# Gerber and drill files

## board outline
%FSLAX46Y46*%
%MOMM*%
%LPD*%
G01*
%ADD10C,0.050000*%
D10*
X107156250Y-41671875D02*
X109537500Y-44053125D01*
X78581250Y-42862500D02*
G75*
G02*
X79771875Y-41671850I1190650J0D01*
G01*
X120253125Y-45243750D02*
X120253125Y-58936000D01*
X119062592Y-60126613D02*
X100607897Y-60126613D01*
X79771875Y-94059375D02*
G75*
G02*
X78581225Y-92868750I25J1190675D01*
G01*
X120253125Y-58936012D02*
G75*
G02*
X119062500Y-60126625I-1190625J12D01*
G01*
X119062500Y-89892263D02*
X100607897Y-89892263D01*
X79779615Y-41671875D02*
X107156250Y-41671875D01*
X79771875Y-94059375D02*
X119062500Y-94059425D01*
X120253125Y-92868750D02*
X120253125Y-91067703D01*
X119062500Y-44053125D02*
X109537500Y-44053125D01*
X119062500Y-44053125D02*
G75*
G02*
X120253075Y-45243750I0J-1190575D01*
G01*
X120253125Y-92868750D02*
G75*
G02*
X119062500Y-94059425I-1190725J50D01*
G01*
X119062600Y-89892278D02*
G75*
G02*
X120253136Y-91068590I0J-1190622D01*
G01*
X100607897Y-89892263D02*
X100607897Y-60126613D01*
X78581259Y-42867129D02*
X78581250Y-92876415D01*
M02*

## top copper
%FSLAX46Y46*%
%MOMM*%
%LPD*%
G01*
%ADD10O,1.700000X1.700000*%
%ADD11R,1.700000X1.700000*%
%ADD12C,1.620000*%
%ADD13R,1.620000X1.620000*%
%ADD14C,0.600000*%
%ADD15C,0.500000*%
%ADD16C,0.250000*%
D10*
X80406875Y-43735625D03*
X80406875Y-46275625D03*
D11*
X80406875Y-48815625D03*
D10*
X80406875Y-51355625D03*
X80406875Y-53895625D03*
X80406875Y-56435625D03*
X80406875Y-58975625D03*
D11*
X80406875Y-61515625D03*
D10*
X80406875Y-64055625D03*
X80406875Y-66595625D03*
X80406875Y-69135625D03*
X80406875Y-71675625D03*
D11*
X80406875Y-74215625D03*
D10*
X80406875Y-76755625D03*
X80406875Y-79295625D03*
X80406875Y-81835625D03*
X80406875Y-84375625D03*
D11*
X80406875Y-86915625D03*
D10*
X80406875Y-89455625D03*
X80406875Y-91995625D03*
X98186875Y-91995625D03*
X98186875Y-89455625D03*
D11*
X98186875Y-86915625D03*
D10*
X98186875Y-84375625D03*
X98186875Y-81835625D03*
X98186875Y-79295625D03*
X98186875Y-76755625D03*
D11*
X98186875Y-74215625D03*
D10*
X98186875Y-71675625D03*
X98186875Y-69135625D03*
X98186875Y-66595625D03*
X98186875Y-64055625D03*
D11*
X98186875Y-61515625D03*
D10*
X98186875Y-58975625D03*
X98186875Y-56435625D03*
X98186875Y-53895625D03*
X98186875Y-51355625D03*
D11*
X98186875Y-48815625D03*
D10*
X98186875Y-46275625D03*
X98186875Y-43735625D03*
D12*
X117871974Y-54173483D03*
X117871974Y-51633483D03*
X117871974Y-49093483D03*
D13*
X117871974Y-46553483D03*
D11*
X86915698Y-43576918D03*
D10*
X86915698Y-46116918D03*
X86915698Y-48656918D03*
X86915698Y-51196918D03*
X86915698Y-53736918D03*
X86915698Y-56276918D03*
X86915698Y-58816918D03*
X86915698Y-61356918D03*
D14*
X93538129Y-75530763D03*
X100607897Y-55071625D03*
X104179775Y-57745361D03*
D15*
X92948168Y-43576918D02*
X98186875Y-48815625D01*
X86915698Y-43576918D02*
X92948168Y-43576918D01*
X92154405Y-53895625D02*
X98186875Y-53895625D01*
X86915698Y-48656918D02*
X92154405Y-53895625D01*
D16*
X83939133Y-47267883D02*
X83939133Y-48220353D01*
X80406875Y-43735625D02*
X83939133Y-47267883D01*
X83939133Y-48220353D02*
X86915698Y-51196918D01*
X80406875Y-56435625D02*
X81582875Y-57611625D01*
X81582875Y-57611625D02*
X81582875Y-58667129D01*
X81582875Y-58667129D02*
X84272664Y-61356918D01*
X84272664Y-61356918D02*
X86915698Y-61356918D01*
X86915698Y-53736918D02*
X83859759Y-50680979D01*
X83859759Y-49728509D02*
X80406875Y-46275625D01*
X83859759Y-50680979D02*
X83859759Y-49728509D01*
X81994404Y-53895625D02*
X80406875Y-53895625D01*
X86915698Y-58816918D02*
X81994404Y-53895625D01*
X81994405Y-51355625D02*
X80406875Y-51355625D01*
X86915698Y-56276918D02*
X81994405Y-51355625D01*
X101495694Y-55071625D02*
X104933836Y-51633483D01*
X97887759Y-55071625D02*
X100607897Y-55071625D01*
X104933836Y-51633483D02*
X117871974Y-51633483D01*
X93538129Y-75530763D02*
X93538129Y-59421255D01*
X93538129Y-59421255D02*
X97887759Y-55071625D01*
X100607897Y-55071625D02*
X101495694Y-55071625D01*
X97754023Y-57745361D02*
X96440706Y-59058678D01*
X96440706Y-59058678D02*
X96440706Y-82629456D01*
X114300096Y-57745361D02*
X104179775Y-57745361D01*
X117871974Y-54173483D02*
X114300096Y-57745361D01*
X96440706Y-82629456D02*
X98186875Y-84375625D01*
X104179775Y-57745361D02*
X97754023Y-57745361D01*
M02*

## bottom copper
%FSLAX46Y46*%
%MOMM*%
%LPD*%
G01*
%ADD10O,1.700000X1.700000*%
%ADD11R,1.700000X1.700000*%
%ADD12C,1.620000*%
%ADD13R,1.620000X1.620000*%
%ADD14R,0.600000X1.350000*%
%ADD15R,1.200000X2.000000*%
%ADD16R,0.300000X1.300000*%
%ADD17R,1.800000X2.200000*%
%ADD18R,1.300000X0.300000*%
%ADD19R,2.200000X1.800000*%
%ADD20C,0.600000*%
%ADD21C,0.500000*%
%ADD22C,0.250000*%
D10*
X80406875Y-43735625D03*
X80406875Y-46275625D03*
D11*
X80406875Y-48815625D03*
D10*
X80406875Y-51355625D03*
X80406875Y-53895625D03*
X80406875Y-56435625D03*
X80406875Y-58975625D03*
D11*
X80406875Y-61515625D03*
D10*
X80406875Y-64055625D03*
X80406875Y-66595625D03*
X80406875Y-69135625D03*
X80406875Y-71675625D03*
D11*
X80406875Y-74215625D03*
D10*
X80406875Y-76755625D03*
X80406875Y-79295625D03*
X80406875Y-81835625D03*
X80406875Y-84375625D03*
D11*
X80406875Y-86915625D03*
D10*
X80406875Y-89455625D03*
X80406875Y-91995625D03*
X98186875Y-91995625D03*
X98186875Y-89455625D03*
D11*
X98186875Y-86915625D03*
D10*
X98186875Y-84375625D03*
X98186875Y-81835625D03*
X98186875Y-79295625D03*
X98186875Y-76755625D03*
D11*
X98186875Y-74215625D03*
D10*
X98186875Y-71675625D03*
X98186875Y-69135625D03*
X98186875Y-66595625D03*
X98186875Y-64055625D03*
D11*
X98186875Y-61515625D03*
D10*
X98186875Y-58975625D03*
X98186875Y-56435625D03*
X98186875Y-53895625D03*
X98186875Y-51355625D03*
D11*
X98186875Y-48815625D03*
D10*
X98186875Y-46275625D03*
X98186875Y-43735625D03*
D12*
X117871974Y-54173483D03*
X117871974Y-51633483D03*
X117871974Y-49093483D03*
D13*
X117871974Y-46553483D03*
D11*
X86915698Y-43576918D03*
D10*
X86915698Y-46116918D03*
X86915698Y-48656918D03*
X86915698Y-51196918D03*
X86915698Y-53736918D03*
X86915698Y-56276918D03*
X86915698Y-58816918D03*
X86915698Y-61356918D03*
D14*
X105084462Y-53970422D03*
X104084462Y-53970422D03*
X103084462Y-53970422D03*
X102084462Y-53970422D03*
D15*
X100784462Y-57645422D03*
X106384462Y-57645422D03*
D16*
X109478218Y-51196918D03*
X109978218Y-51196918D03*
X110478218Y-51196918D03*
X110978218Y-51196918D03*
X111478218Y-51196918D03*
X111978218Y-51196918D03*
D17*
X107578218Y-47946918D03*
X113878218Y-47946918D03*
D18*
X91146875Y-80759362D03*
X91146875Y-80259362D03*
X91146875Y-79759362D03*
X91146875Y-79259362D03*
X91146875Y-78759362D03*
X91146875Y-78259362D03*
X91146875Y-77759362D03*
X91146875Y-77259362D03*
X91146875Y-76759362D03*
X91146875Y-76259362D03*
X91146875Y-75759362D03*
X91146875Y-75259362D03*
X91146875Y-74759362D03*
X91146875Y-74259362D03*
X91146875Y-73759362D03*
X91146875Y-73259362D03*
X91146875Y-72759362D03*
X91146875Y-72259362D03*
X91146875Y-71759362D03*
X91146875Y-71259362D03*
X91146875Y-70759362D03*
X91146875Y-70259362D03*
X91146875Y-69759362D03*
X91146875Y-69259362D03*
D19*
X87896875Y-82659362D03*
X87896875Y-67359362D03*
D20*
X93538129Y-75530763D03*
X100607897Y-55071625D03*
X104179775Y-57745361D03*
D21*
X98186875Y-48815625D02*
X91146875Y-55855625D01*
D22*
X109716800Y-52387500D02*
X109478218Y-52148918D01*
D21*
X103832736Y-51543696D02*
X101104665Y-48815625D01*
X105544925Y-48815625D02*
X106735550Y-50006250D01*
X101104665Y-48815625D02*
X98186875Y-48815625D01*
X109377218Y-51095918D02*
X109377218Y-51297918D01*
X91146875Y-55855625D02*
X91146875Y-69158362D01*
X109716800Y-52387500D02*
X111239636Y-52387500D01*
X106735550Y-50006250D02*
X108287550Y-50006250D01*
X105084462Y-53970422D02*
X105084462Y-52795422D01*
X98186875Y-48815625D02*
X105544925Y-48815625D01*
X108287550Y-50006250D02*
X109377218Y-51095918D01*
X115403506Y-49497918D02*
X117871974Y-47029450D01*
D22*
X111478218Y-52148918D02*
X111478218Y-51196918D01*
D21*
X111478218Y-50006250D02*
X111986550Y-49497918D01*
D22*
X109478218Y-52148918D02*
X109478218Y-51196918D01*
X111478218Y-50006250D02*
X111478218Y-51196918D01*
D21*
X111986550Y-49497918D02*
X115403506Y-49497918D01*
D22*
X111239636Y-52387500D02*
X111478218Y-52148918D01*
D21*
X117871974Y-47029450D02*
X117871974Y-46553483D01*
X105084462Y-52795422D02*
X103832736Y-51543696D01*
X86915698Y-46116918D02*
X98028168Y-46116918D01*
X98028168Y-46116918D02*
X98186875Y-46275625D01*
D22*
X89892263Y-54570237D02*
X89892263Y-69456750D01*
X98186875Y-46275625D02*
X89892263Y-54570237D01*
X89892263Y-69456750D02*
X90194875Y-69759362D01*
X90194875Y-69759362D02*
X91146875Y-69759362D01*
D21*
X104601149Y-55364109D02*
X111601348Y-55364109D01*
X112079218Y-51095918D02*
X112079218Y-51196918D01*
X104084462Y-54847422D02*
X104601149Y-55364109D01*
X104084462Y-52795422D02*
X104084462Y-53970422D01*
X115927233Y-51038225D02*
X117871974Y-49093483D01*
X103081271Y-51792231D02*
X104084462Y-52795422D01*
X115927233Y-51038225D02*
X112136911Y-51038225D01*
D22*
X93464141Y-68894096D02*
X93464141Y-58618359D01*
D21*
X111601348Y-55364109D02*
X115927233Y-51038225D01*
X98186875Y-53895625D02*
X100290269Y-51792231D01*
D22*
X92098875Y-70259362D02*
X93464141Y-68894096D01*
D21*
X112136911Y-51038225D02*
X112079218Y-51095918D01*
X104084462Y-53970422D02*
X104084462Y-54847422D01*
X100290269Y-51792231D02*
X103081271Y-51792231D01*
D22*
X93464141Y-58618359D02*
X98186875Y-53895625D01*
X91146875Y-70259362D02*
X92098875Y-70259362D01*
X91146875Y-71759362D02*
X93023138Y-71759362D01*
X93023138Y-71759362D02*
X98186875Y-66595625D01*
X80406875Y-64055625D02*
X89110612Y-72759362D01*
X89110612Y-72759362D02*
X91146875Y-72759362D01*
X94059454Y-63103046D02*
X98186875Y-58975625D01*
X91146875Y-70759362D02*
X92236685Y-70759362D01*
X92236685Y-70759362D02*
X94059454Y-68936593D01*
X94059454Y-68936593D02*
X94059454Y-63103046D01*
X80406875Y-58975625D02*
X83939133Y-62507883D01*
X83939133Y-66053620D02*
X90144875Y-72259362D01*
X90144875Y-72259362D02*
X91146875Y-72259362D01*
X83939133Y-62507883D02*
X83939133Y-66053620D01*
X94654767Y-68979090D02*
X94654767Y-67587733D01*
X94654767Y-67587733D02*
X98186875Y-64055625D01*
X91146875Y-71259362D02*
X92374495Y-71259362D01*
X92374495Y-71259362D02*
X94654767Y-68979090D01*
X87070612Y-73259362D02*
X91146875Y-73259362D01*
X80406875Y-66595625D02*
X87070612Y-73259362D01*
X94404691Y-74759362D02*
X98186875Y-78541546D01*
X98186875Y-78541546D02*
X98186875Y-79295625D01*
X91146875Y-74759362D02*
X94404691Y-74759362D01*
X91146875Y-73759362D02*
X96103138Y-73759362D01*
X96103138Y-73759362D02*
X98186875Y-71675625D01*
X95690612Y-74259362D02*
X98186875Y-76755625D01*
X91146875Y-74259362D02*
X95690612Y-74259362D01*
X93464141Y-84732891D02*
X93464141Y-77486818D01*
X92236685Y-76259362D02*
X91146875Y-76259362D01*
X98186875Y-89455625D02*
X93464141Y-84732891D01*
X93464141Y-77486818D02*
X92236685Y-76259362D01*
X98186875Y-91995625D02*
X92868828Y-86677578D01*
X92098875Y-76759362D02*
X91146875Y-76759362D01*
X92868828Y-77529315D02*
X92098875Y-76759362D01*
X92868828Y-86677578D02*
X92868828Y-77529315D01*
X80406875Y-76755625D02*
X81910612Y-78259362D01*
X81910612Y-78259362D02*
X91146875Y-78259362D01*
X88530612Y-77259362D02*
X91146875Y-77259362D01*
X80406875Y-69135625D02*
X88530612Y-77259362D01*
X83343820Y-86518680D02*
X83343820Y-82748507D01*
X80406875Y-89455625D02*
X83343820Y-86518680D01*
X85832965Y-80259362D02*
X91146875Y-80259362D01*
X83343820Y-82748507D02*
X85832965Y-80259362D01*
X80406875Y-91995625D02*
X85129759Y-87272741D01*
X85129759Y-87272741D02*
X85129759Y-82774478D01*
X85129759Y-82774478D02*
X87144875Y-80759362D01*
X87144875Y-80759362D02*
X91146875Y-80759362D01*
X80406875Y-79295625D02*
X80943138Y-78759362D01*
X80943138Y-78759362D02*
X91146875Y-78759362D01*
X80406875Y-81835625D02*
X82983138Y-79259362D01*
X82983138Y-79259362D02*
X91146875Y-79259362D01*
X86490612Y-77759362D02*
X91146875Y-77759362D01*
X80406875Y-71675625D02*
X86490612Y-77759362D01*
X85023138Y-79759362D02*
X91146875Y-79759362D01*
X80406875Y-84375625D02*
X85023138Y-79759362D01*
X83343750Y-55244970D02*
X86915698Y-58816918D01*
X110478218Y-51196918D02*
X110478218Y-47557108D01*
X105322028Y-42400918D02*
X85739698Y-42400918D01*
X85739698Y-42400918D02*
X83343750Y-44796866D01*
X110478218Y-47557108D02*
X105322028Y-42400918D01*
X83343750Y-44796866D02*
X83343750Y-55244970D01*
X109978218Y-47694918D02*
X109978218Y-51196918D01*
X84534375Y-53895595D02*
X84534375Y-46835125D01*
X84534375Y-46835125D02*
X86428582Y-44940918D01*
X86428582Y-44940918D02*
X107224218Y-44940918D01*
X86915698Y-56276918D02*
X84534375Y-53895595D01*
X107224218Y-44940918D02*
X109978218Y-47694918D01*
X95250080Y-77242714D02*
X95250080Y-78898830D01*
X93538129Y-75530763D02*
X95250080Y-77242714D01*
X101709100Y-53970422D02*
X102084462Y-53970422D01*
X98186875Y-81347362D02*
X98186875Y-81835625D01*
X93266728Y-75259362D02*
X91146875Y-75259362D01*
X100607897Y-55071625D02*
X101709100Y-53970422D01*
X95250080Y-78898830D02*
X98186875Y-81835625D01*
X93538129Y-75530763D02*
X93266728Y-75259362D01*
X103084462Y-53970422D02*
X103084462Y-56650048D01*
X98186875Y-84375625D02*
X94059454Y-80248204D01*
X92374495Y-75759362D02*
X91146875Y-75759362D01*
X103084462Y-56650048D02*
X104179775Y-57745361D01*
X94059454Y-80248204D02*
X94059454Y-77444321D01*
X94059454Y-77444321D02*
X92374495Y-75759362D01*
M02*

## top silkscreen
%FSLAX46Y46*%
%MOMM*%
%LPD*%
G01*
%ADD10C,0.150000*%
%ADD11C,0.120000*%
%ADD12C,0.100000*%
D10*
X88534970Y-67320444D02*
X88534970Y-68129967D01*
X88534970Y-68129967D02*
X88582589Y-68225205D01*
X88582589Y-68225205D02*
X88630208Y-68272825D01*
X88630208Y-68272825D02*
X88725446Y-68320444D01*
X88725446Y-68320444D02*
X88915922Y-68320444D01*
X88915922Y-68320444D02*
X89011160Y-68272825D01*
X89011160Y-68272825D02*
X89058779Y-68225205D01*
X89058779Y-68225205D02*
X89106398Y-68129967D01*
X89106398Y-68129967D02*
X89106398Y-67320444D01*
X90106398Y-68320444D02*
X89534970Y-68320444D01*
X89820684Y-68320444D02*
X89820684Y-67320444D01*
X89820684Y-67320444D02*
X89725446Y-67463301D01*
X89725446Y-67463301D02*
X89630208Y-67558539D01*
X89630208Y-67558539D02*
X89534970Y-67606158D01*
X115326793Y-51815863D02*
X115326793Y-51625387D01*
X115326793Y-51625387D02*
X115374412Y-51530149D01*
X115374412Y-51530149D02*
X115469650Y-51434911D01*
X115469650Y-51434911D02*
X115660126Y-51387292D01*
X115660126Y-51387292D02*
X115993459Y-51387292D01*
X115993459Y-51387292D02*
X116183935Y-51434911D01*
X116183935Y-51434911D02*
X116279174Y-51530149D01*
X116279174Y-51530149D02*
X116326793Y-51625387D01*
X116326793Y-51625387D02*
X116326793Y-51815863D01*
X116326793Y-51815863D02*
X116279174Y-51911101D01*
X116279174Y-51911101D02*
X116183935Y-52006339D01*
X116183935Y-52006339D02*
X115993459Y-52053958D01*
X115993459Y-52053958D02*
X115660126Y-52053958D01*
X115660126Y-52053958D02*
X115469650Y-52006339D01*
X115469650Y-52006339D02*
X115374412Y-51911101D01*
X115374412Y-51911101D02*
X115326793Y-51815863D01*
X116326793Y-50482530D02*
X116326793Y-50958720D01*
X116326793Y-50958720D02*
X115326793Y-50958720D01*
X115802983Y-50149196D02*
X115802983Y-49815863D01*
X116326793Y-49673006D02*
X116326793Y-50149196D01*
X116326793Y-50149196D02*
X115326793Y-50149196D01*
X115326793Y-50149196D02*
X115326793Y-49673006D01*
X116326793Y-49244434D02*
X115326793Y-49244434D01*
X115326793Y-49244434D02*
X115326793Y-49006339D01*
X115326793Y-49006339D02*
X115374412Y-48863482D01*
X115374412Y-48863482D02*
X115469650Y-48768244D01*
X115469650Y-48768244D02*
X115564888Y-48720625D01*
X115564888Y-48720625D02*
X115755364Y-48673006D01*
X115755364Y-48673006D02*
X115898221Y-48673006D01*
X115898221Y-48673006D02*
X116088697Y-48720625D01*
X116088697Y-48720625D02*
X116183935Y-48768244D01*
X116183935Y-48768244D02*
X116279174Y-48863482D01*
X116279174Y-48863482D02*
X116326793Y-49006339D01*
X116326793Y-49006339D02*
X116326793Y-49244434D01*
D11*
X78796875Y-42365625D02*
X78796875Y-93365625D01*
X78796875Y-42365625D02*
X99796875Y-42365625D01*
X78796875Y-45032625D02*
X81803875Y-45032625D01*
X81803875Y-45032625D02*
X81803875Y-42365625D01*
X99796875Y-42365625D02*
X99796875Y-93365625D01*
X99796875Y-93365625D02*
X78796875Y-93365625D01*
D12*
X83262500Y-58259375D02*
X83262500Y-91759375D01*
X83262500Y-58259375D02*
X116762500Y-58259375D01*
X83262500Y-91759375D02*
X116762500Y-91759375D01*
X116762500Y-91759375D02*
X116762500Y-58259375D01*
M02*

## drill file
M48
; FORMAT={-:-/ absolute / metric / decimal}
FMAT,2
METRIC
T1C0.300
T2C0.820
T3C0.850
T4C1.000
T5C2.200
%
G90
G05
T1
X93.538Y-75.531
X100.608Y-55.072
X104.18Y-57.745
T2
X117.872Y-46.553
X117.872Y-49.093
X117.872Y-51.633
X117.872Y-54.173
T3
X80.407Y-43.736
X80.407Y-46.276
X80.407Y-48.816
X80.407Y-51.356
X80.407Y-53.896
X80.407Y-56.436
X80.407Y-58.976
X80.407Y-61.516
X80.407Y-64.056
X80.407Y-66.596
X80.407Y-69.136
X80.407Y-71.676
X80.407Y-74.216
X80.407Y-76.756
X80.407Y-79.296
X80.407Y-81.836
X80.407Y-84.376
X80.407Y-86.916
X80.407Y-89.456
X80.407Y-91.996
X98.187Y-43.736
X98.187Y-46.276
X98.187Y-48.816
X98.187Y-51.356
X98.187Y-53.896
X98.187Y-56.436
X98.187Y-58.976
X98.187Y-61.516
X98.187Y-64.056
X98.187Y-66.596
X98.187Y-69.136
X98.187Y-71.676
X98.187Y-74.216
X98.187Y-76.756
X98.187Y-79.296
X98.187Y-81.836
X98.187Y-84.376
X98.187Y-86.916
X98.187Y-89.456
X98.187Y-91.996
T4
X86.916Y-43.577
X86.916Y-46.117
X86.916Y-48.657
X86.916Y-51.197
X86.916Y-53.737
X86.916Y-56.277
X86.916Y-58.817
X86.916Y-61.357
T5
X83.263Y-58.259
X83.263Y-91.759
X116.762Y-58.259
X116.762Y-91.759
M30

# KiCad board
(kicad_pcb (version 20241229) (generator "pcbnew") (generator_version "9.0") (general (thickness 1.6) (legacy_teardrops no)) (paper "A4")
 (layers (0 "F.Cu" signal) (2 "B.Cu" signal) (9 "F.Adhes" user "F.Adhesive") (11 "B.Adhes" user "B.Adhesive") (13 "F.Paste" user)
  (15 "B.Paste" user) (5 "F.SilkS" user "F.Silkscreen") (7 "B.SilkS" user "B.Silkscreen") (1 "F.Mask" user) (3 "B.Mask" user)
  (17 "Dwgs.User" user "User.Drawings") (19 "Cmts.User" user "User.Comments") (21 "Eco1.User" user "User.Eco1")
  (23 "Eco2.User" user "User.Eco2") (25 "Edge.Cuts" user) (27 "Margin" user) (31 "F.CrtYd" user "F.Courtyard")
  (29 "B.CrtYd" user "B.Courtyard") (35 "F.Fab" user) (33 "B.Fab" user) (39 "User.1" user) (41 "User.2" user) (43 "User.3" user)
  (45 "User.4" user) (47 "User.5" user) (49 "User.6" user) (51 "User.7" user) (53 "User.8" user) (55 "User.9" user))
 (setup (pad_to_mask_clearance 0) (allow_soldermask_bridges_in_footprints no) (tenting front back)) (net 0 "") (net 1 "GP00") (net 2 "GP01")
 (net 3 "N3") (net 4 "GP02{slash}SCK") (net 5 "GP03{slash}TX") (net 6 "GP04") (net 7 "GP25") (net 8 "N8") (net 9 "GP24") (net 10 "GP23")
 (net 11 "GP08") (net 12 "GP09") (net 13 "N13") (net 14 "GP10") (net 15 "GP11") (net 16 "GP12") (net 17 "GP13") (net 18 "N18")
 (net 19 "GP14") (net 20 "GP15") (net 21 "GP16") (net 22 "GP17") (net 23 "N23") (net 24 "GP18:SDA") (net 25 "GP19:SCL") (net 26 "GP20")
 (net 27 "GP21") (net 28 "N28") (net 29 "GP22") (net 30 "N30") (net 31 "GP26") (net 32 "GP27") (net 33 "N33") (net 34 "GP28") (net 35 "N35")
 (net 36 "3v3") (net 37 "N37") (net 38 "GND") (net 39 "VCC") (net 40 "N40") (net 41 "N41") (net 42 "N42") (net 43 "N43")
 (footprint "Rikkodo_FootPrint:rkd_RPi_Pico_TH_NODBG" (layer "F.Cu") (at 89.296875 67.865625)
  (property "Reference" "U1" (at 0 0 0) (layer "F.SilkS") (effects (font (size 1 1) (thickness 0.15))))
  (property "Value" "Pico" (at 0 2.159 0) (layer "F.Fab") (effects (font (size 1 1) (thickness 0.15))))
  (fp_line (start -10.5 -25.5) (end -10.5 25.5) (stroke (width 0.12) (type solid)) (layer "F.SilkS"))
  (fp_line (start -10.5 -25.5) (end 10.5 -25.5) (stroke (width 0.12) (type solid)) (layer "F.SilkS"))
  (fp_line (start -10.5 -22.833) (end -7.493 -22.833) (stroke (width 0.12) (type solid)) (layer "F.SilkS"))
  (fp_line (start -7.493 -22.833) (end -7.493 -25.5) (stroke (width 0.12) (type solid)) (layer "F.SilkS"))
  (fp_line (start 10.5 -25.5) (end 10.5 25.5) (stroke (width 0.12) (type solid)) (layer "F.SilkS"))
  (fp_line (start 10.5 25.5) (end -10.5 25.5) (stroke (width 0.12) (type solid)) (layer "F.SilkS"))
  (pad "1" thru_hole oval (at -8.89 -24.13) (size 1.7 1.7) (drill 0.85) (layers "*.Cu" "*.Mask") (remove_unused_layers no) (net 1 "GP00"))
  (pad "2" thru_hole oval (at -8.89 -21.59) (size 1.7 1.7) (drill 0.85) (layers "*.Cu" "*.Mask") (remove_unused_layers no) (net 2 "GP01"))
  (pad "3" thru_hole rect (at -8.89 -19.05) (size 1.7 1.7) (drill 0.85) (layers "*.Cu" "*.Mask") (remove_unused_layers no) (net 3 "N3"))
  (pad "4" thru_hole oval (at -8.89 -16.51) (size 1.7 1.7) (drill 0.85) (layers "*.Cu" "*.Mask") (remove_unused_layers no)
   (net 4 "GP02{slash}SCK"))
  (pad "5" thru_hole oval (at -8.89 -13.97) (size 1.7 1.7) (drill 0.85) (layers "*.Cu" "*.Mask") (remove_unused_layers no)
   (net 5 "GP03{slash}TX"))
  (pad "6" thru_hole oval (at -8.89 -11.43) (size 1.7 1.7) (drill 0.85) (layers "*.Cu" "*.Mask") (remove_unused_layers no) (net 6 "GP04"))
  (pad "7" thru_hole oval (at -8.89 -8.89) (size 1.7 1.7) (drill 0.85) (layers "*.Cu" "*.Mask") (remove_unused_layers no) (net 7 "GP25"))
  (pad "8" thru_hole rect (at -8.89 -6.35) (size 1.7 1.7) (drill 0.85) (layers "*.Cu" "*.Mask") (remove_unused_layers no) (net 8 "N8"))
  (pad "9" thru_hole oval (at -8.89 -3.81) (size 1.7 1.7) (drill 0.85) (layers "*.Cu" "*.Mask") (remove_unused_layers no) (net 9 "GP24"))
  (pad "10" thru_hole oval (at -8.89 -1.27) (size 1.7 1.7) (drill 0.85) (layers "*.Cu" "*.Mask") (remove_unused_layers no) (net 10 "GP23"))
  (pad "11" thru_hole oval (at -8.89 1.27) (size 1.7 1.7) (drill 0.85) (layers "*.Cu" "*.Mask") (remove_unused_layers no) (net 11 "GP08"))
  (pad "12" thru_hole oval (at -8.89 3.81) (size 1.7 1.7) (drill 0.85) (layers "*.Cu" "*.Mask") (remove_unused_layers no) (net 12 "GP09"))
  (pad "13" thru_hole rect (at -8.89 6.35) (size 1.7 1.7) (drill 0.85) (layers "*.Cu" "*.Mask") (remove_unused_layers no) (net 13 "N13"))
  (pad "14" thru_hole oval (at -8.89 8.89) (size 1.7 1.7) (drill 0.85) (layers "*.Cu" "*.Mask") (remove_unused_layers no) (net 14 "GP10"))
  (pad "15" thru_hole oval (at -8.89 11.43) (size 1.7 1.7) (drill 0.85) (layers "*.Cu" "*.Mask") (remove_unused_layers no) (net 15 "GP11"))
  (pad "16" thru_hole oval (at -8.89 13.97) (size 1.7 1.7) (drill 0.85) (layers "*.Cu" "*.Mask") (remove_unused_layers no) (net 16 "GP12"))
  (pad "17" thru_hole oval (at -8.89 16.51) (size 1.7 1.7) (drill 0.85) (layers "*.Cu" "*.Mask") (remove_unused_layers no) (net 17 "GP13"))
  (pad "18" thru_hole rect (at -8.89 19.05) (size 1.7 1.7) (drill 0.85) (layers "*.Cu" "*.Mask") (remove_unused_layers no) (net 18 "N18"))
  (pad "19" thru_hole oval (at -8.89 21.59) (size 1.7 1.7) (drill 0.85) (layers "*.Cu" "*.Mask") (remove_unused_layers no) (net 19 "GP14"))
  (pad "20" thru_hole oval (at -8.89 24.13) (size 1.7 1.7) (drill 0.85) (layers "*.Cu" "*.Mask") (remove_unused_layers no) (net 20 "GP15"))
  (pad "21" thru_hole oval (at 8.89 24.13) (size 1.7 1.7) (drill 0.85) (layers "*.Cu" "*.Mask") (remove_unused_layers no) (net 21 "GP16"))
  (pad "22" thru_hole oval (at 8.89 21.59) (size 1.7 1.7) (drill 0.85) (layers "*.Cu" "*.Mask") (remove_unused_layers no) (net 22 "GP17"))
  (pad "23" thru_hole rect (at 8.89 19.05) (size 1.7 1.7) (drill 0.85) (layers "*.Cu" "*.Mask") (remove_unused_layers no) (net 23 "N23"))
  (pad "24" thru_hole oval (at 8.89 16.51) (size 1.7 1.7) (drill 0.85) (layers "*.Cu" "*.Mask") (remove_unused_layers no)
   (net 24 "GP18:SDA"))
  (pad "25" thru_hole oval (at 8.89 13.97) (size 1.7 1.7) (drill 0.85) (layers "*.Cu" "*.Mask") (remove_unused_layers no)
   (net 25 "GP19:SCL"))
  (pad "26" thru_hole oval (at 8.89 11.43) (size 1.7 1.7) (drill 0.85) (layers "*.Cu" "*.Mask") (remove_unused_layers no) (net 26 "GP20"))
  (pad "27" thru_hole oval (at 8.89 8.89) (size 1.7 1.7) (drill 0.85) (layers "*.Cu" "*.Mask") (remove_unused_layers no) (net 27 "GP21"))
  (pad "28" thru_hole rect (at 8.89 6.35) (size 1.7 1.7) (drill 0.85) (layers "*.Cu" "*.Mask") (remove_unused_layers no) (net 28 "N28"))
  (pad "29" thru_hole oval (at 8.89 3.81) (size 1.7 1.7) (drill 0.85) (layers "*.Cu" "*.Mask") (remove_unused_layers no) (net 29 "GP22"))
  (pad "30" thru_hole oval (at 8.89 1.27) (size 1.7 1.7) (drill 0.85) (layers "*.Cu" "*.Mask") (remove_unused_layers no) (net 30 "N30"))
  (pad "31" thru_hole oval (at 8.89 -1.27) (size 1.7 1.7) (drill 0.85) (layers "*.Cu" "*.Mask") (remove_unused_layers no) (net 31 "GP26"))
  (pad "32" thru_hole oval (at 8.89 -3.81) (size 1.7 1.7) (drill 0.85) (layers "*.Cu" "*.Mask") (remove_unused_layers no) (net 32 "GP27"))
  (pad "33" thru_hole rect (at 8.89 -6.35) (size 1.7 1.7) (drill 0.85) (layers "*.Cu" "*.Mask") (remove_unused_layers no) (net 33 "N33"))
  (pad "34" thru_hole oval (at 8.89 -8.89) (size 1.7 1.7) (drill 0.85) (layers "*.Cu" "*.Mask") (remove_unused_layers no) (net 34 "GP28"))
  (pad "35" thru_hole oval (at 8.89 -11.43) (size 1.7 1.7) (drill 0.85) (layers "*.Cu" "*.Mask") (remove_unused_layers no) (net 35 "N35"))
  (pad "36" thru_hole oval (at 8.89 -13.97) (size 1.7 1.7) (drill 0.85) (layers "*.Cu" "*.Mask") (remove_unused_layers no) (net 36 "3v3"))
  (pad "37" thru_hole oval (at 8.89 -16.51) (size 1.7 1.7) (drill 0.85) (layers "*.Cu" "*.Mask") (remove_unused_layers no) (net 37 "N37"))
  (pad "38" thru_hole rect (at 8.89 -19.05) (size 1.7 1.7) (drill 0.85) (layers "*.Cu" "*.Mask") (remove_unused_layers no) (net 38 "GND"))
  (pad "39" thru_hole oval (at 8.89 -21.59) (size 1.7 1.7) (drill 0.85) (layers "*.Cu" "*.Mask") (remove_unused_layers no) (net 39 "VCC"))
  (pad "40" thru_hole oval (at 8.89 -24.13) (size 1.7 1.7) (drill 0.85) (layers "*.Cu" "*.Mask") (remove_unused_layers no) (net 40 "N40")))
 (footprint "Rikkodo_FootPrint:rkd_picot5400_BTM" (layer "F.Cu") (at 100.0125 75.009375)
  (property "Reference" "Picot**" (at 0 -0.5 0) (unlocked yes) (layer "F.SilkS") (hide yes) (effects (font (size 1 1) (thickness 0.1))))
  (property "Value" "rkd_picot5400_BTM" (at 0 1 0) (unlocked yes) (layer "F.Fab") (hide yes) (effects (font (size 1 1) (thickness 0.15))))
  (fp_line (start -16.75 -16.75) (end -16.75 16.75) (stroke (width 0.1) (type default)) (layer "F.SilkS"))
  (fp_line (start -16.75 -16.75) (end 16.75 -16.75) (stroke (width 0.1) (type default)) (layer "F.SilkS"))
  (fp_line (start -16.75 16.75) (end 16.75 16.75) (stroke (width 0.1) (type default)) (layer "F.SilkS"))
  (fp_line (start 16.75 16.75) (end 16.75 -16.75) (stroke (width 0.1) (type default)) (layer "F.SilkS"))
  (pad "" np_thru_hole circle (at -16.75 -16.75) (size 2.2 2.2) (drill 2.2) (layers "*.Cu" "*.Mask"))
  (pad "" np_thru_hole circle (at -16.75 16.75) (size 2.2 2.2) (drill 2.2) (layers "*.Cu" "*.Mask"))
  (pad "" np_thru_hole circle (at 16.75 -16.75) (size 2.2 2.2) (drill 2.2) (layers "*.Cu" "*.Mask"))
  (pad "" np_thru_hole circle (at 16.75 16.75) (size 2.2 2.2) (drill 2.2) (layers "*.Cu" "*.Mask")))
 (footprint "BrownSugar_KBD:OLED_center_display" (layer "F.Cu") (at 99.371974 50.363483 90)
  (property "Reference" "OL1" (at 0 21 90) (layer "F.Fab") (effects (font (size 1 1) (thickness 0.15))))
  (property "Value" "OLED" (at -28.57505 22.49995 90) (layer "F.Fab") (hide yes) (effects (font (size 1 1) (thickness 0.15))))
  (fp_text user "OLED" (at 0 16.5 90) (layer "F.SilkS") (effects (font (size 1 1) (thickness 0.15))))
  (pad "1" thru_hole circle (at -3.81 18.5 90) (size 1.62 1.62) (drill 0.82) (layers "*.Cu" "*.Mask") (remove_unused_layers no)
   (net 24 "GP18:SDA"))
  (pad "2" thru_hole circle (at -1.27 18.5 90) (size 1.62 1.62) (drill 0.82) (layers "*.Cu" "*.Mask") (remove_unused_layers no)
   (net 25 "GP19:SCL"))
  (pad "3" thru_hole circle (at 1.27 18.5 90) (size 1.62 1.62) (drill 0.82) (layers "*.Cu" "*.Mask") (remove_unused_layers no)
   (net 36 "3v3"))
  (pad "4" thru_hole rect (at 3.81 18.5 90) (size 1.62 1.62) (drill 0.82) (layers "*.Cu" "*.Mask") (remove_unused_layers no) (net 38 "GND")))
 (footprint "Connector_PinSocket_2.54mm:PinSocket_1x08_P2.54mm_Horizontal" (layer "B.Cu") (at 86.915698 43.576918 180)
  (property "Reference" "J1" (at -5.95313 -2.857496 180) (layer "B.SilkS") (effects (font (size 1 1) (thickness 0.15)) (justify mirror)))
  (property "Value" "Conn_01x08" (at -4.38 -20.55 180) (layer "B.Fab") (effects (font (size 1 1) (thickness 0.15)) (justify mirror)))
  (pad "1" thru_hole rect (at 0 0 180) (size 1.7 1.7) (drill 1) (layers "*.Cu" "*.Mask") (remove_unused_layers no) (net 38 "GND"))
  (pad "2" thru_hole oval (at 0 -2.54 180) (size 1.7 1.7) (drill 1) (layers "*.Cu" "*.Mask") (remove_unused_layers no) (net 39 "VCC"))
  (pad "3" thru_hole oval (at 0 -5.08 180) (size 1.7 1.7) (drill 1) (layers "*.Cu" "*.Mask") (remove_unused_layers no) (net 36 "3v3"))
  (pad "4" thru_hole oval (at 0 -7.62 180) (size 1.7 1.7) (drill 1) (layers "*.Cu" "*.Mask") (remove_unused_layers no) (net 1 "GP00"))
  (pad "5" thru_hole oval (at 0 -10.16 180) (size 1.7 1.7) (drill 1) (layers "*.Cu" "*.Mask") (remove_unused_layers no) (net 2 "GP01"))
  (pad "6" thru_hole oval (at 0 -12.7 180) (size 1.7 1.7) (drill 1) (layers "*.Cu" "*.Mask") (remove_unused_layers no)
   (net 4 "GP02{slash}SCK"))
  (pad "7" thru_hole oval (at 0 -15.24 180) (size 1.7 1.7) (drill 1) (layers "*.Cu" "*.Mask") (remove_unused_layers no)
   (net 5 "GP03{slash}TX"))
  (pad "8" thru_hole oval (at 0 -17.78 180) (size 1.7 1.7) (drill 1) (layers "*.Cu" "*.Mask") (remove_unused_layers no) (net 6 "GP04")))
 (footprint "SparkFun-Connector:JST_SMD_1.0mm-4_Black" (layer "B.Cu") (at 103.584462 53.970422 180)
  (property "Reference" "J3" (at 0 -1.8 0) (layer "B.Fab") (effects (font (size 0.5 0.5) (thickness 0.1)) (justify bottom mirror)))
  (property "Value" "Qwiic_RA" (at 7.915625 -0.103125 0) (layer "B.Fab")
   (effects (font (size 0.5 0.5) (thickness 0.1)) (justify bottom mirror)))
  (pad "1" smd rect (at -1.5 0 180) (size 0.6 1.35) (layers "B.Cu" "B.Mask" "B.Paste") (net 38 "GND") (thermal_bridge_angle 0))
  (pad "2" smd rect (at -0.5 0 180) (size 0.6 1.35) (layers "B.Cu" "B.Mask" "B.Paste") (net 36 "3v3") (thermal_bridge_angle 0))
  (pad "3" smd rect (at 0.5 0 180) (size 0.6 1.35) (layers "B.Cu" "B.Mask" "B.Paste") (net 24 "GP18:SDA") (thermal_bridge_angle 0))
  (pad "4" smd rect (at 1.5 0 180) (size 0.6 1.35) (layers "B.Cu" "B.Mask" "B.Paste") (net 25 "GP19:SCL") (thermal_bridge_angle 0))
  (pad "NC1" smd rect (at 2.8 -3.675 180) (size 1.2 2) (layers "B.Cu" "B.Mask" "B.Paste") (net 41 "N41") (thermal_bridge_angle 0))
  (pad "NC2" smd rect (at -2.8 -3.675 180) (size 1.2 2) (layers "B.Cu" "B.Mask" "B.Paste") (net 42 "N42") (thermal_bridge_angle 0)))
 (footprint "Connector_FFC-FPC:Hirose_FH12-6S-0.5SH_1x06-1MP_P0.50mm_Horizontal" (layer "B.Cu") (at 110.728218 49.346918)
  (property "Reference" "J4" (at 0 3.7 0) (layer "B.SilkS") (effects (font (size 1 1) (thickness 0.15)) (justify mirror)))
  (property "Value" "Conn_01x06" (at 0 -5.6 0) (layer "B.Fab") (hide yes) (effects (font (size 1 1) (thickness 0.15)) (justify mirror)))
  (pad "1" smd rect (at -1.25 1.85) (size 0.3 1.3) (layers "B.Cu" "B.Mask" "B.Paste") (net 38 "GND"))
  (pad "2" smd rect (at -0.75 1.85) (size 0.3 1.3) (layers "B.Cu" "B.Mask" "B.Paste") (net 4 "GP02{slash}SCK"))
  (pad "3" smd rect (at -0.25 1.85) (size 0.3 1.3) (layers "B.Cu" "B.Mask" "B.Paste") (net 5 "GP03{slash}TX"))
  (pad "4" smd rect (at 0.25 1.85) (size 0.3 1.3) (layers "B.Cu" "B.Mask" "B.Paste") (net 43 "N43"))
  (pad "5" smd rect (at 0.75 1.85) (size 0.3 1.3) (layers "B.Cu" "B.Mask" "B.Paste") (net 38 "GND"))
  (pad "6" smd rect (at 1.25 1.85) (size 0.3 1.3) (layers "B.Cu" "B.Mask" "B.Paste") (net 36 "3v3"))
  (pad "MP" smd rect (at -3.15 -1.4) (size 1.8 2.2) (layers "B.Cu" "B.Mask" "B.Paste"))
  (pad "MP" smd rect (at 3.15 -1.4) (size 1.8 2.2) (layers "B.Cu" "B.Mask" "B.Paste")))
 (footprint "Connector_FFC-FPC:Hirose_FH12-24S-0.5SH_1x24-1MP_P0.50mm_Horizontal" (layer "B.Cu") (at 89.296875 75.009362 90)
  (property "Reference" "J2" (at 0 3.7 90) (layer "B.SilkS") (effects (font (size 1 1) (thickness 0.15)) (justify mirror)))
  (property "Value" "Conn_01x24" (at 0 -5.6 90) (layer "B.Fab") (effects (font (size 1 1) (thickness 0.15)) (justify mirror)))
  (pad "1" smd rect (at -5.75 1.85 90) (size 0.3 1.3) (layers "B.Cu" "B.Mask" "B.Paste") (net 20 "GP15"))
  (pad "2" smd rect (at -5.25 1.85 90) (size 0.3 1.3) (layers "B.Cu" "B.Mask" "B.Paste") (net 19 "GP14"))
  (pad "3" smd rect (at -4.75 1.85 90) (size 0.3 1.3) (layers "B.Cu" "B.Mask" "B.Paste") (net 17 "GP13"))
  (pad "4" smd rect (at -4.25 1.85 90) (size 0.3 1.3) (layers "B.Cu" "B.Mask" "B.Paste") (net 16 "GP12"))
  (pad "5" smd rect (at -3.75 1.85 90) (size 0.3 1.3) (layers "B.Cu" "B.Mask" "B.Paste") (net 15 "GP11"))
  (pad "6" smd rect (at -3.25 1.85 90) (size 0.3 1.3) (layers "B.Cu" "B.Mask" "B.Paste") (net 14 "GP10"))
  (pad "7" smd rect (at -2.75 1.85 90) (size 0.3 1.3) (layers "B.Cu" "B.Mask" "B.Paste") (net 12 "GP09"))
  (pad "8" smd rect (at -2.25 1.85 90) (size 0.3 1.3) (layers "B.Cu" "B.Mask" "B.Paste") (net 11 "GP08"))
  (pad "9" smd rect (at -1.75 1.85 90) (size 0.3 1.3) (layers "B.Cu" "B.Mask" "B.Paste") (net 21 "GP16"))
  (pad "10" smd rect (at -1.25 1.85 90) (size 0.3 1.3) (layers "B.Cu" "B.Mask" "B.Paste") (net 22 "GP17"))
  (pad "11" smd rect (at -0.75 1.85 90) (size 0.3 1.3) (layers "B.Cu" "B.Mask" "B.Paste") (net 24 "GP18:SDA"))
  (pad "12" smd rect (at -0.25 1.85 90) (size 0.3 1.3) (layers "B.Cu" "B.Mask" "B.Paste") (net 25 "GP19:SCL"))
  (pad "13" smd rect (at 0.25 1.85 90) (size 0.3 1.3) (layers "B.Cu" "B.Mask" "B.Paste") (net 26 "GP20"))
  (pad "14" smd rect (at 0.75 1.85 90) (size 0.3 1.3) (layers "B.Cu" "B.Mask" "B.Paste") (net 27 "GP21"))
  (pad "15" smd rect (at 1.25 1.85 90) (size 0.3 1.3) (layers "B.Cu" "B.Mask" "B.Paste") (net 29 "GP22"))
  (pad "16" smd rect (at 1.75 1.85 90) (size 0.3 1.3) (layers "B.Cu" "B.Mask" "B.Paste") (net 10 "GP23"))
  (pad "17" smd rect (at 2.25 1.85 90) (size 0.3 1.3) (layers "B.Cu" "B.Mask" "B.Paste") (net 9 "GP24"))
  (pad "18" smd rect (at 2.75 1.85 90) (size 0.3 1.3) (layers "B.Cu" "B.Mask" "B.Paste") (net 7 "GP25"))
  (pad "19" smd rect (at 3.25 1.85 90) (size 0.3 1.3) (layers "B.Cu" "B.Mask" "B.Paste") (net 31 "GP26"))
  (pad "20" smd rect (at 3.75 1.85 90) (size 0.3 1.3) (layers "B.Cu" "B.Mask" "B.Paste") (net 32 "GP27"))
  (pad "21" smd rect (at 4.25 1.85 90) (size 0.3 1.3) (layers "B.Cu" "B.Mask" "B.Paste") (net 34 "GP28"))
  (pad "22" smd rect (at 4.75 1.85 90) (size 0.3 1.3) (layers "B.Cu" "B.Mask" "B.Paste") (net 36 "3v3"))
  (pad "23" smd rect (at 5.25 1.85 90) (size 0.3 1.3) (layers "B.Cu" "B.Mask" "B.Paste") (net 39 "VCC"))
  (pad "24" smd rect (at 5.75 1.85 90) (size 0.3 1.3) (layers "B.Cu" "B.Mask" "B.Paste") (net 38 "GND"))
  (pad "MP" smd rect (at -7.65 -1.4 90) (size 1.8 2.2) (layers "B.Cu" "B.Mask" "B.Paste"))
  (pad "MP" smd rect (at 7.65 -1.4 90) (size 1.8 2.2) (layers "B.Cu" "B.Mask" "B.Paste")))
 (gr_line (start 107.15625 41.671875) (end 109.5375 44.053125) (stroke (width 0.05) (type default)) (layer "Edge.Cuts"))
 (gr_arc (start 78.58125 42.8625) (mid 78.929974 42.020592) (end 79.771875 41.671875) (stroke (width 0.05) (type default))
  (layer "Edge.Cuts"))
 (gr_line (start 120.253125 45.24375) (end 120.253125 58.936) (stroke (width 0.05) (type default)) (layer "Edge.Cuts"))
 (gr_line (start 119.062592 60.126613) (end 100.607897 60.126613) (stroke (width 0.05) (type default)) (layer "Edge.Cuts"))
 (gr_arc (start 79.771875 94.059375) (mid 78.929974 93.710643) (end 78.58125 92.86875) (stroke (width 0.05) (type default))
  (layer "Edge.Cuts"))
 (gr_arc (start 120.253125 58.936012) (mid 119.904395 59.777903) (end 119.0625 60.126637) (stroke (width 0.05) (type default))
  (layer "Edge.Cuts"))
 (gr_line (start 119.0625 89.892263) (end 100.607897 89.892263) (stroke (width 0.05) (type default)) (layer "Edge.Cuts"))
 (gr_line (start 79.779615 41.671875) (end 107.15625 41.671875) (stroke (width 0.05) (type default)) (layer "Edge.Cuts"))
 (gr_line (start 79.771875 94.059375) (end 119.0625 94.059425) (stroke (width 0.05) (type default)) (layer "Edge.Cuts"))
 (gr_line (start 120.253125 92.86875) (end 120.253125 91.067703) (stroke (width 0.05) (type default)) (layer "Edge.Cuts"))
 (gr_line (start 119.0625 44.053125) (end 109.5375 44.053125) (stroke (width 0.05) (type default)) (layer "Edge.Cuts"))
 (gr_arc (start 119.0625 44.053125) (mid 119.904417 44.401848) (end 120.253125 45.24375) (stroke (width 0.05) (type default))
  (layer "Edge.Cuts"))
 (gr_arc (start 120.253125 92.86875) (mid 119.904381 93.710617) (end 119.0625 94.059375) (stroke (width 0.05) (type default))
  (layer "Edge.Cuts"))
 (gr_arc (start 119.0626 89.892278) (mid 119.899422 90.235959) (end 120.253125 91.06859) (stroke (width 0.05) (type default))
  (layer "Edge.Cuts"))
 (gr_line (start 100.607897 89.892263) (end 100.607897 60.126613) (stroke (width 0.05) (type default)) (layer "Edge.Cuts"))
 (gr_line (start 78.581259 42.867129) (end 78.58125 92.876415) (stroke (width 0.05) (type default)) (layer "Edge.Cuts"))
 (segment (start 92.948168 43.576918) (end 98.186875 48.815625) (width 0.5) (layer "F.Cu") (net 38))
 (segment (start 86.915698 43.576918) (end 92.948168 43.576918) (width 0.5) (layer "F.Cu") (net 38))
 (segment (start 98.186875 48.815625) (end 91.146875 55.855625) (width 0.5) (layer "B.Cu") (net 38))
 (segment (start 109.7168 52.3875) (end 109.478218 52.148918) (width 0.25) (layer "B.Cu") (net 38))
 (segment (start 103.832736 51.543696) (end 101.104665 48.815625) (width 0.5) (layer "B.Cu") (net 38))
 (segment (start 105.544925 48.815625) (end 106.73555 50.00625) (width 0.5) (layer "B.Cu") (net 38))
 (segment (start 101.104665 48.815625) (end 98.186875 48.815625) (width 0.5) (layer "B.Cu") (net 38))
 (segment (start 109.377218 51.095918) (end 109.377218 51.297918) (width 0.5) (layer "B.Cu") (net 38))
 (segment (start 91.146875 55.855625) (end 91.146875 69.158362) (width 0.5) (layer "B.Cu") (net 38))
 (segment (start 109.7168 52.3875) (end 111.239636 52.3875) (width 0.5) (layer "B.Cu") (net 38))
 (segment (start 106.73555 50.00625) (end 108.28755 50.00625) (width 0.5) (layer "B.Cu") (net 38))
 (segment (start 105.084462 53.970422) (end 105.084462 52.795422) (width 0.5) (layer "B.Cu") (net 38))
 (segment (start 98.186875 48.815625) (end 105.544925 48.815625) (width 0.5) (layer "B.Cu") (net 38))
 (segment (start 108.28755 50.00625) (end 109.377218 51.095918) (width 0.5) (layer "B.Cu") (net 38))
 (segment (start 115.403506 49.497918) (end 117.871974 47.02945) (width 0.5) (layer "B.Cu") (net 38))
 (segment (start 111.478218 52.148918) (end 111.478218 51.196918) (width 0.25) (layer "B.Cu") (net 38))
 (segment (start 111.478218 50.00625) (end 111.98655 49.497918) (width 0.5) (layer "B.Cu") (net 38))
 (segment (start 109.478218 52.148918) (end 109.478218 51.196918) (width 0.25) (layer "B.Cu") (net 38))
 (segment (start 111.478218 50.00625) (end 111.478218 51.196918) (width 0.25) (layer "B.Cu") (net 38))
 (segment (start 111.98655 49.497918) (end 115.403506 49.497918) (width 0.5) (layer "B.Cu") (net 38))
 (segment (start 111.239636 52.3875) (end 111.478218 52.148918) (width 0.25) (layer "B.Cu") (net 38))
 (segment (start 117.871974 47.02945) (end 117.871974 46.553483) (width 0.5) (layer "B.Cu") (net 38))
 (segment (start 105.084462 52.795422) (end 103.832736 51.543696) (width 0.5) (layer "B.Cu") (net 38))
 (segment (start 86.915698 46.116918) (end 98.028168 46.116918) (width 0.5) (layer "B.Cu") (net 39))
 (segment (start 98.028168 46.116918) (end 98.186875 46.275625) (width 0.5) (layer "B.Cu") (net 39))
 (segment (start 89.892263 54.570237) (end 89.892263 69.45675) (width 0.25) (layer "B.Cu") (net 39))
 (segment (start 98.186875 46.275625) (end 89.892263 54.570237) (width 0.25) (layer "B.Cu") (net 39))
 (segment (start 89.892263 69.45675) (end 90.194875 69.759362) (width 0.25) (layer "B.Cu") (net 39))
 (segment (start 90.194875 69.759362) (end 91.146875 69.759362) (width 0.25) (layer "B.Cu") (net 39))
 (segment (start 92.154405 53.895625) (end 98.186875 53.895625) (width 0.5) (layer "F.Cu") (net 36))
 (segment (start 86.915698 48.656918) (end 92.154405 53.895625) (width 0.5) (layer "F.Cu") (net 36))
 (segment (start 104.601149 55.364109) (end 111.601348 55.364109) (width 0.5) (layer "B.Cu") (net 36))
 (segment (start 112.079218 51.095918) (end 112.079218 51.196918) (width 0.5) (layer "B.Cu") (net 36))
 (segment (start 104.084462 54.847422) (end 104.601149 55.364109) (width 0.5) (layer "B.Cu") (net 36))
 (segment (start 104.084462 52.795422) (end 104.084462 53.970422) (width 0.5) (layer "B.Cu") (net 36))
 (segment (start 115.927233 51.038225) (end 117.871974 49.093483) (width 0.5) (layer "B.Cu") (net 36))
 (segment (start 103.081271 51.792231) (end 104.084462 52.795422) (width 0.5) (layer "B.Cu") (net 36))
 (segment (start 115.927233 51.038225) (end 112.136911 51.038225) (width 0.5) (layer "B.Cu") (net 36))
 (segment (start 93.464141 68.894096) (end 93.464141 58.618359) (width 0.25) (layer "B.Cu") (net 36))
 (segment (start 111.601348 55.364109) (end 115.927233 51.038225) (width 0.5) (layer "B.Cu") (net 36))
 (segment (start 98.186875 53.895625) (end 100.290269 51.792231) (width 0.5) (layer "B.Cu") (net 36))
 (segment (start 92.098875 70.259362) (end 93.464141 68.894096) (width 0.25) (layer "B.Cu") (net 36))
 (segment (start 112.136911 51.038225) (end 112.079218 51.095918) (width 0.5) (layer "B.Cu") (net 36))
 (segment (start 104.084462 53.970422) (end 104.084462 54.847422) (width 0.5) (layer "B.Cu") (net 36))
 (segment (start 100.290269 51.792231) (end 103.081271 51.792231) (width 0.5) (layer "B.Cu") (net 36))
 (segment (start 93.464141 58.618359) (end 98.186875 53.895625) (width 0.25) (layer "B.Cu") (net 36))
 (segment (start 91.146875 70.259362) (end 92.098875 70.259362) (width 0.25) (layer "B.Cu") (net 36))
 (segment (start 91.146875 71.759362) (end 93.023138 71.759362) (width 0.25) (layer "B.Cu") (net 31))
 (segment (start 93.023138 71.759362) (end 98.186875 66.595625) (width 0.25) (layer "B.Cu") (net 31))
 (segment (start 80.406875 64.055625) (end 89.110612 72.759362) (width 0.25) (layer "B.Cu") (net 9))
 (segment (start 89.110612 72.759362) (end 91.146875 72.759362) (width 0.25) (layer "B.Cu") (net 9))
 (segment (start 94.059454 63.103046) (end 98.186875 58.975625) (width 0.25) (layer "B.Cu") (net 34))
 (segment (start 91.146875 70.759362) (end 92.236685 70.759362) (width 0.25) (layer "B.Cu") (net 34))
 (segment (start 92.236685 70.759362) (end 94.059454 68.936593) (width 0.25) (layer "B.Cu") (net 34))
 (segment (start 94.059454 68.936593) (end 94.059454 63.103046) (width 0.25) (layer "B.Cu") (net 34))
 (segment (start 80.406875 58.975625) (end 83.939133 62.507883) (width 0.25) (layer "B.Cu") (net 7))
 (segment (start 83.939133 66.05362) (end 90.144875 72.259362) (width 0.25) (layer "B.Cu") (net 7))
 (segment (start 90.144875 72.259362) (end 91.146875 72.259362) (width 0.25) (layer "B.Cu") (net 7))
 (segment (start 83.939133 62.507883) (end 83.939133 66.05362) (width 0.25) (layer "B.Cu") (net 7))
 (segment (start 94.654767 68.97909) (end 94.654767 67.587733) (width 0.25) (layer "B.Cu") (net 32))
 (segment (start 94.654767 67.587733) (end 98.186875 64.055625) (width 0.25) (layer "B.Cu") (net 32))
 (segment (start 91.146875 71.259362) (end 92.374495 71.259362) (width 0.25) (layer "B.Cu") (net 32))
 (segment (start 92.374495 71.259362) (end 94.654767 68.97909) (width 0.25) (layer "B.Cu") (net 32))
 (segment (start 87.070612 73.259362) (end 91.146875 73.259362) (width 0.25) (layer "B.Cu") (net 10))
 (segment (start 80.406875 66.595625) (end 87.070612 73.259362) (width 0.25) (layer "B.Cu") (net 10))
 (segment (start 94.404691 74.759362) (end 98.186875 78.541546) (width 0.25) (layer "B.Cu") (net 26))
 (segment (start 98.186875 78.541546) (end 98.186875 79.295625) (width 0.25) (layer "B.Cu") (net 26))
 (segment (start 91.146875 74.759362) (end 94.404691 74.759362) (width 0.25) (layer "B.Cu") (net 26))
 (segment (start 91.146875 73.759362) (end 96.103138 73.759362) (width 0.25) (layer "B.Cu") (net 29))
 (segment (start 96.103138 73.759362) (end 98.186875 71.675625) (width 0.25) (layer "B.Cu") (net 29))
 (segment (start 95.690612 74.259362) (end 98.186875 76.755625) (width 0.25) (layer "B.Cu") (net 27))
 (segment (start 91.146875 74.259362) (end 95.690612 74.259362) (width 0.25) (layer "B.Cu") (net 27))
 (segment (start 93.464141 84.732891) (end 93.464141 77.486818) (width 0.25) (layer "B.Cu") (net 22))
 (segment (start 92.236685 76.259362) (end 91.146875 76.259362) (width 0.25) (layer "B.Cu") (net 22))
 (segment (start 98.186875 89.455625) (end 93.464141 84.732891) (width 0.25) (layer "B.Cu") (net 22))
 (segment (start 93.464141 77.486818) (end 92.236685 76.259362) (width 0.25) (layer "B.Cu") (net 22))
 (segment (start 98.186875 91.995625) (end 92.868828 86.677578) (width 0.25) (layer "B.Cu") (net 21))
 (segment (start 92.098875 76.759362) (end 91.146875 76.759362) (width 0.25) (layer "B.Cu") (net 21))
 (segment (start 92.868828 77.529315) (end 92.098875 76.759362) (width 0.25) (layer "B.Cu") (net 21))
 (segment (start 92.868828 86.677578) (end 92.868828 77.529315) (width 0.25) (layer "B.Cu") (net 21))
 (segment (start 80.406875 76.755625) (end 81.910612 78.259362) (width 0.25) (layer "B.Cu") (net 14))
 (segment (start 81.910612 78.259362) (end 91.146875 78.259362) (width 0.25) (layer "B.Cu") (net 14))
 (segment (start 88.530612 77.259362) (end 91.146875 77.259362) (width 0.25) (layer "B.Cu") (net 11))
 (segment (start 80.406875 69.135625) (end 88.530612 77.259362) (width 0.25) (layer "B.Cu") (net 11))
 (segment (start 83.34382 86.51868) (end 83.34382 82.748507) (width 0.25) (layer "B.Cu") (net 19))
 (segment (start 80.406875 89.455625) (end 83.34382 86.51868) (width 0.25) (layer "B.Cu") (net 19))
 (segment (start 85.832965 80.259362) (end 91.146875 80.259362) (width 0.25) (layer "B.Cu") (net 19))
 (segment (start 83.34382 82.748507) (end 85.832965 80.259362) (width 0.25) (layer "B.Cu") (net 19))
 (segment (start 80.406875 91.995625) (end 85.129759 87.272741) (width 0.25) (layer "B.Cu") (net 20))
 (segment (start 85.129759 87.272741) (end 85.129759 82.774478) (width 0.25) (layer "B.Cu") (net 20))
 (segment (start 85.129759 82.774478) (end 87.144875 80.759362) (width 0.25) (layer "B.Cu") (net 20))
 (segment (start 87.144875 80.759362) (end 91.146875 80.759362) (width 0.25) (layer "B.Cu") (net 20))
 (segment (start 80.406875 79.295625) (end 80.943138 78.759362) (width 0.25) (layer "B.Cu") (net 15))
 (segment (start 80.943138 78.759362) (end 91.146875 78.759362) (width 0.25) (layer "B.Cu") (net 15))
 (segment (start 80.406875 81.835625) (end 82.983138 79.259362) (width 0.25) (layer "B.Cu") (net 16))
 (segment (start 82.983138 79.259362) (end 91.146875 79.259362) (width 0.25) (layer "B.Cu") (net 16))
 (segment (start 86.490612 77.759362) (end 91.146875 77.759362) (width 0.25) (layer "B.Cu") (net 12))
 (segment (start 80.406875 71.675625) (end 86.490612 77.759362) (width 0.25) (layer "B.Cu") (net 12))
 (segment (start 85.023138 79.759362) (end 91.146875 79.759362) (width 0.25) (layer "B.Cu") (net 17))
 (segment (start 80.406875 84.375625) (end 85.023138 79.759362) (width 0.25) (layer "B.Cu") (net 17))
 (segment (start 83.939133 47.267883) (end 83.939133 48.220353) (width 0.25) (layer "F.Cu") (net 1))
 (segment (start 80.406875 43.735625) (end 83.939133 47.267883) (width 0.25) (layer "F.Cu") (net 1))
 (segment (start 83.939133 48.220353) (end 86.915698 51.196918) (width 0.25) (layer "F.Cu") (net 1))
 (segment (start 80.406875 56.435625) (end 81.582875 57.611625) (width 0.25) (layer "F.Cu") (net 6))
 (segment (start 81.582875 57.611625) (end 81.582875 58.667129) (width 0.25) (layer "F.Cu") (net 6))
 (segment (start 81.582875 58.667129) (end 84.272664 61.356918) (width 0.25) (layer "F.Cu") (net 6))
 (segment (start 84.272664 61.356918) (end 86.915698 61.356918) (width 0.25) (layer "F.Cu") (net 6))
 (segment (start 86.915698 53.736918) (end 83.859759 50.680979) (width 0.25) (layer "F.Cu") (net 2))
 (segment (start 83.859759 49.728509) (end 80.406875 46.275625) (width 0.25) (layer "F.Cu") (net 2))
 (segment (start 83.859759 50.680979) (end 83.859759 49.728509) (width 0.25) (layer "F.Cu") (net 2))
 (segment (start 81.994404 53.895625) (end 80.406875 53.895625) (width 0.25) (layer "F.Cu") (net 5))
 (segment (start 86.915698 58.816918) (end 81.994404 53.895625) (width 0.25) (layer "F.Cu") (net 5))
 (segment (start 83.34375 55.24497) (end 86.915698 58.816918) (width 0.25) (layer "B.Cu") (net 5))
 (segment (start 110.478218 51.196918) (end 110.478218 47.557108) (width 0.25) (layer "B.Cu") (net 5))
 (segment (start 105.322028 42.400918) (end 85.739698 42.400918) (width 0.25) (layer "B.Cu") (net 5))
 (segment (start 85.739698 42.400918) (end 83.34375 44.796866) (width 0.25) (layer "B.Cu") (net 5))
 (segment (start 110.478218 47.557108) (end 105.322028 42.400918) (width 0.25) (layer "B.Cu") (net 5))
 (segment (start 83.34375 44.796866) (end 83.34375 55.24497) (width 0.25) (layer "B.Cu") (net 5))
 (segment (start 81.994405 51.355625) (end 80.406875 51.355625) (width 0.25) (layer "F.Cu") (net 4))
 (segment (start 86.915698 56.276918) (end 81.994405 51.355625) (width 0.25) (layer "F.Cu") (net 4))
 (segment (start 109.978218 47.694918) (end 109.978218 51.196918) (width 0.25) (layer "B.Cu") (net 4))
 (segment (start 84.534375 53.895595) (end 84.534375 46.835125) (width 0.25) (layer "B.Cu") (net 4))
 (segment (start 84.534375 46.835125) (end 86.428582 44.940918) (width 0.25) (layer "B.Cu") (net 4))
 (segment (start 86.428582 44.940918) (end 107.224218 44.940918) (width 0.25) (layer "B.Cu") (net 4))
 (segment (start 86.915698 56.276918) (end 84.534375 53.895595) (width 0.25) (layer "B.Cu") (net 4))
 (segment (start 107.224218 44.940918) (end 109.978218 47.694918) (width 0.25) (layer "B.Cu") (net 4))
 (segment (start 101.495694 55.071625) (end 104.933836 51.633483) (width 0.25) (layer "F.Cu") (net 25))
 (segment (start 97.887759 55.071625) (end 100.607897 55.071625) (width 0.25) (layer "F.Cu") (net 25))
 (segment (start 104.933836 51.633483) (end 117.871974 51.633483) (width 0.25) (layer "F.Cu") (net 25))
 (segment (start 93.538129 75.530763) (end 93.538129 59.421255) (width 0.25) (layer "F.Cu") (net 25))
 (segment (start 93.538129 59.421255) (end 97.887759 55.071625) (width 0.25) (layer "F.Cu") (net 25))
 (segment (start 100.607897 55.071625) (end 101.495694 55.071625) (width 0.25) (layer "F.Cu") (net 25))
 (via (at 93.538129 75.530763) (size 0.6) (drill 0.3) (layers "F.Cu" "B.Cu") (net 25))
 (via (at 100.607897 55.071625) (size 0.6) (drill 0.3) (layers "F.Cu" "B.Cu") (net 25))
 (segment (start 95.25008 77.242714) (end 95.25008 78.89883) (width 0.25) (layer "B.Cu") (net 25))
 (segment (start 93.538129 75.530763) (end 95.25008 77.242714) (width 0.25) (layer "B.Cu") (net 25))
 (segment (start 101.7091 53.970422) (end 102.084462 53.970422) (width 0.25) (layer "B.Cu") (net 25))
 (segment (start 98.186875 81.347362) (end 98.186875 81.835625) (width 0.25) (layer "B.Cu") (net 25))
 (segment (start 93.266728 75.259362) (end 91.146875 75.259362) (width 0.25) (layer "B.Cu") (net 25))
 (segment (start 100.607897 55.071625) (end 101.7091 53.970422) (width 0.25) (layer "B.Cu") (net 25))
 (segment (start 95.25008 78.89883) (end 98.186875 81.835625) (width 0.25) (layer "B.Cu") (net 25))
 (segment (start 93.538129 75.530763) (end 93.266728 75.259362) (width 0.25) (layer "B.Cu") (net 25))
 (segment (start 97.754023 57.745361) (end 96.440706 59.058678) (width 0.25) (layer "F.Cu") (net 24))
 (segment (start 96.440706 59.058678) (end 96.440706 82.629456) (width 0.25) (layer "F.Cu") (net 24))
 (segment (start 114.300096 57.745361) (end 104.179775 57.745361) (width 0.25) (layer "F.Cu") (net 24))
 (segment (start 117.871974 54.173483) (end 114.300096 57.745361) (width 0.25) (layer "F.Cu") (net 24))
 (segment (start 96.440706 82.629456) (end 98.186875 84.375625) (width 0.25) (layer "F.Cu") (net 24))
 (segment (start 104.179775 57.745361) (end 97.754023 57.745361) (width 0.25) (layer "F.Cu") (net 24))
 (via (at 104.179775 57.745361) (size 0.6) (drill 0.3) (layers "F.Cu" "B.Cu") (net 24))
 (segment (start 103.084462 53.970422) (end 103.084462 56.650048) (width 0.25) (layer "B.Cu") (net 24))
 (segment (start 98.186875 84.375625) (end 94.059454 80.248204) (width 0.25) (layer "B.Cu") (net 24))
 (segment (start 92.374495 75.759362) (end 91.146875 75.759362) (width 0.25) (layer "B.Cu") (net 24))
 (segment (start 103.084462 56.650048) (end 104.179775 57.745361) (width 0.25) (layer "B.Cu") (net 24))
 (segment (start 94.059454 80.248204) (end 94.059454 77.444321) (width 0.25) (layer "B.Cu") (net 24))
 (segment (start 94.059454 77.444321) (end 92.374495 75.759362) (width 0.25) (layer "B.Cu") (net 24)))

